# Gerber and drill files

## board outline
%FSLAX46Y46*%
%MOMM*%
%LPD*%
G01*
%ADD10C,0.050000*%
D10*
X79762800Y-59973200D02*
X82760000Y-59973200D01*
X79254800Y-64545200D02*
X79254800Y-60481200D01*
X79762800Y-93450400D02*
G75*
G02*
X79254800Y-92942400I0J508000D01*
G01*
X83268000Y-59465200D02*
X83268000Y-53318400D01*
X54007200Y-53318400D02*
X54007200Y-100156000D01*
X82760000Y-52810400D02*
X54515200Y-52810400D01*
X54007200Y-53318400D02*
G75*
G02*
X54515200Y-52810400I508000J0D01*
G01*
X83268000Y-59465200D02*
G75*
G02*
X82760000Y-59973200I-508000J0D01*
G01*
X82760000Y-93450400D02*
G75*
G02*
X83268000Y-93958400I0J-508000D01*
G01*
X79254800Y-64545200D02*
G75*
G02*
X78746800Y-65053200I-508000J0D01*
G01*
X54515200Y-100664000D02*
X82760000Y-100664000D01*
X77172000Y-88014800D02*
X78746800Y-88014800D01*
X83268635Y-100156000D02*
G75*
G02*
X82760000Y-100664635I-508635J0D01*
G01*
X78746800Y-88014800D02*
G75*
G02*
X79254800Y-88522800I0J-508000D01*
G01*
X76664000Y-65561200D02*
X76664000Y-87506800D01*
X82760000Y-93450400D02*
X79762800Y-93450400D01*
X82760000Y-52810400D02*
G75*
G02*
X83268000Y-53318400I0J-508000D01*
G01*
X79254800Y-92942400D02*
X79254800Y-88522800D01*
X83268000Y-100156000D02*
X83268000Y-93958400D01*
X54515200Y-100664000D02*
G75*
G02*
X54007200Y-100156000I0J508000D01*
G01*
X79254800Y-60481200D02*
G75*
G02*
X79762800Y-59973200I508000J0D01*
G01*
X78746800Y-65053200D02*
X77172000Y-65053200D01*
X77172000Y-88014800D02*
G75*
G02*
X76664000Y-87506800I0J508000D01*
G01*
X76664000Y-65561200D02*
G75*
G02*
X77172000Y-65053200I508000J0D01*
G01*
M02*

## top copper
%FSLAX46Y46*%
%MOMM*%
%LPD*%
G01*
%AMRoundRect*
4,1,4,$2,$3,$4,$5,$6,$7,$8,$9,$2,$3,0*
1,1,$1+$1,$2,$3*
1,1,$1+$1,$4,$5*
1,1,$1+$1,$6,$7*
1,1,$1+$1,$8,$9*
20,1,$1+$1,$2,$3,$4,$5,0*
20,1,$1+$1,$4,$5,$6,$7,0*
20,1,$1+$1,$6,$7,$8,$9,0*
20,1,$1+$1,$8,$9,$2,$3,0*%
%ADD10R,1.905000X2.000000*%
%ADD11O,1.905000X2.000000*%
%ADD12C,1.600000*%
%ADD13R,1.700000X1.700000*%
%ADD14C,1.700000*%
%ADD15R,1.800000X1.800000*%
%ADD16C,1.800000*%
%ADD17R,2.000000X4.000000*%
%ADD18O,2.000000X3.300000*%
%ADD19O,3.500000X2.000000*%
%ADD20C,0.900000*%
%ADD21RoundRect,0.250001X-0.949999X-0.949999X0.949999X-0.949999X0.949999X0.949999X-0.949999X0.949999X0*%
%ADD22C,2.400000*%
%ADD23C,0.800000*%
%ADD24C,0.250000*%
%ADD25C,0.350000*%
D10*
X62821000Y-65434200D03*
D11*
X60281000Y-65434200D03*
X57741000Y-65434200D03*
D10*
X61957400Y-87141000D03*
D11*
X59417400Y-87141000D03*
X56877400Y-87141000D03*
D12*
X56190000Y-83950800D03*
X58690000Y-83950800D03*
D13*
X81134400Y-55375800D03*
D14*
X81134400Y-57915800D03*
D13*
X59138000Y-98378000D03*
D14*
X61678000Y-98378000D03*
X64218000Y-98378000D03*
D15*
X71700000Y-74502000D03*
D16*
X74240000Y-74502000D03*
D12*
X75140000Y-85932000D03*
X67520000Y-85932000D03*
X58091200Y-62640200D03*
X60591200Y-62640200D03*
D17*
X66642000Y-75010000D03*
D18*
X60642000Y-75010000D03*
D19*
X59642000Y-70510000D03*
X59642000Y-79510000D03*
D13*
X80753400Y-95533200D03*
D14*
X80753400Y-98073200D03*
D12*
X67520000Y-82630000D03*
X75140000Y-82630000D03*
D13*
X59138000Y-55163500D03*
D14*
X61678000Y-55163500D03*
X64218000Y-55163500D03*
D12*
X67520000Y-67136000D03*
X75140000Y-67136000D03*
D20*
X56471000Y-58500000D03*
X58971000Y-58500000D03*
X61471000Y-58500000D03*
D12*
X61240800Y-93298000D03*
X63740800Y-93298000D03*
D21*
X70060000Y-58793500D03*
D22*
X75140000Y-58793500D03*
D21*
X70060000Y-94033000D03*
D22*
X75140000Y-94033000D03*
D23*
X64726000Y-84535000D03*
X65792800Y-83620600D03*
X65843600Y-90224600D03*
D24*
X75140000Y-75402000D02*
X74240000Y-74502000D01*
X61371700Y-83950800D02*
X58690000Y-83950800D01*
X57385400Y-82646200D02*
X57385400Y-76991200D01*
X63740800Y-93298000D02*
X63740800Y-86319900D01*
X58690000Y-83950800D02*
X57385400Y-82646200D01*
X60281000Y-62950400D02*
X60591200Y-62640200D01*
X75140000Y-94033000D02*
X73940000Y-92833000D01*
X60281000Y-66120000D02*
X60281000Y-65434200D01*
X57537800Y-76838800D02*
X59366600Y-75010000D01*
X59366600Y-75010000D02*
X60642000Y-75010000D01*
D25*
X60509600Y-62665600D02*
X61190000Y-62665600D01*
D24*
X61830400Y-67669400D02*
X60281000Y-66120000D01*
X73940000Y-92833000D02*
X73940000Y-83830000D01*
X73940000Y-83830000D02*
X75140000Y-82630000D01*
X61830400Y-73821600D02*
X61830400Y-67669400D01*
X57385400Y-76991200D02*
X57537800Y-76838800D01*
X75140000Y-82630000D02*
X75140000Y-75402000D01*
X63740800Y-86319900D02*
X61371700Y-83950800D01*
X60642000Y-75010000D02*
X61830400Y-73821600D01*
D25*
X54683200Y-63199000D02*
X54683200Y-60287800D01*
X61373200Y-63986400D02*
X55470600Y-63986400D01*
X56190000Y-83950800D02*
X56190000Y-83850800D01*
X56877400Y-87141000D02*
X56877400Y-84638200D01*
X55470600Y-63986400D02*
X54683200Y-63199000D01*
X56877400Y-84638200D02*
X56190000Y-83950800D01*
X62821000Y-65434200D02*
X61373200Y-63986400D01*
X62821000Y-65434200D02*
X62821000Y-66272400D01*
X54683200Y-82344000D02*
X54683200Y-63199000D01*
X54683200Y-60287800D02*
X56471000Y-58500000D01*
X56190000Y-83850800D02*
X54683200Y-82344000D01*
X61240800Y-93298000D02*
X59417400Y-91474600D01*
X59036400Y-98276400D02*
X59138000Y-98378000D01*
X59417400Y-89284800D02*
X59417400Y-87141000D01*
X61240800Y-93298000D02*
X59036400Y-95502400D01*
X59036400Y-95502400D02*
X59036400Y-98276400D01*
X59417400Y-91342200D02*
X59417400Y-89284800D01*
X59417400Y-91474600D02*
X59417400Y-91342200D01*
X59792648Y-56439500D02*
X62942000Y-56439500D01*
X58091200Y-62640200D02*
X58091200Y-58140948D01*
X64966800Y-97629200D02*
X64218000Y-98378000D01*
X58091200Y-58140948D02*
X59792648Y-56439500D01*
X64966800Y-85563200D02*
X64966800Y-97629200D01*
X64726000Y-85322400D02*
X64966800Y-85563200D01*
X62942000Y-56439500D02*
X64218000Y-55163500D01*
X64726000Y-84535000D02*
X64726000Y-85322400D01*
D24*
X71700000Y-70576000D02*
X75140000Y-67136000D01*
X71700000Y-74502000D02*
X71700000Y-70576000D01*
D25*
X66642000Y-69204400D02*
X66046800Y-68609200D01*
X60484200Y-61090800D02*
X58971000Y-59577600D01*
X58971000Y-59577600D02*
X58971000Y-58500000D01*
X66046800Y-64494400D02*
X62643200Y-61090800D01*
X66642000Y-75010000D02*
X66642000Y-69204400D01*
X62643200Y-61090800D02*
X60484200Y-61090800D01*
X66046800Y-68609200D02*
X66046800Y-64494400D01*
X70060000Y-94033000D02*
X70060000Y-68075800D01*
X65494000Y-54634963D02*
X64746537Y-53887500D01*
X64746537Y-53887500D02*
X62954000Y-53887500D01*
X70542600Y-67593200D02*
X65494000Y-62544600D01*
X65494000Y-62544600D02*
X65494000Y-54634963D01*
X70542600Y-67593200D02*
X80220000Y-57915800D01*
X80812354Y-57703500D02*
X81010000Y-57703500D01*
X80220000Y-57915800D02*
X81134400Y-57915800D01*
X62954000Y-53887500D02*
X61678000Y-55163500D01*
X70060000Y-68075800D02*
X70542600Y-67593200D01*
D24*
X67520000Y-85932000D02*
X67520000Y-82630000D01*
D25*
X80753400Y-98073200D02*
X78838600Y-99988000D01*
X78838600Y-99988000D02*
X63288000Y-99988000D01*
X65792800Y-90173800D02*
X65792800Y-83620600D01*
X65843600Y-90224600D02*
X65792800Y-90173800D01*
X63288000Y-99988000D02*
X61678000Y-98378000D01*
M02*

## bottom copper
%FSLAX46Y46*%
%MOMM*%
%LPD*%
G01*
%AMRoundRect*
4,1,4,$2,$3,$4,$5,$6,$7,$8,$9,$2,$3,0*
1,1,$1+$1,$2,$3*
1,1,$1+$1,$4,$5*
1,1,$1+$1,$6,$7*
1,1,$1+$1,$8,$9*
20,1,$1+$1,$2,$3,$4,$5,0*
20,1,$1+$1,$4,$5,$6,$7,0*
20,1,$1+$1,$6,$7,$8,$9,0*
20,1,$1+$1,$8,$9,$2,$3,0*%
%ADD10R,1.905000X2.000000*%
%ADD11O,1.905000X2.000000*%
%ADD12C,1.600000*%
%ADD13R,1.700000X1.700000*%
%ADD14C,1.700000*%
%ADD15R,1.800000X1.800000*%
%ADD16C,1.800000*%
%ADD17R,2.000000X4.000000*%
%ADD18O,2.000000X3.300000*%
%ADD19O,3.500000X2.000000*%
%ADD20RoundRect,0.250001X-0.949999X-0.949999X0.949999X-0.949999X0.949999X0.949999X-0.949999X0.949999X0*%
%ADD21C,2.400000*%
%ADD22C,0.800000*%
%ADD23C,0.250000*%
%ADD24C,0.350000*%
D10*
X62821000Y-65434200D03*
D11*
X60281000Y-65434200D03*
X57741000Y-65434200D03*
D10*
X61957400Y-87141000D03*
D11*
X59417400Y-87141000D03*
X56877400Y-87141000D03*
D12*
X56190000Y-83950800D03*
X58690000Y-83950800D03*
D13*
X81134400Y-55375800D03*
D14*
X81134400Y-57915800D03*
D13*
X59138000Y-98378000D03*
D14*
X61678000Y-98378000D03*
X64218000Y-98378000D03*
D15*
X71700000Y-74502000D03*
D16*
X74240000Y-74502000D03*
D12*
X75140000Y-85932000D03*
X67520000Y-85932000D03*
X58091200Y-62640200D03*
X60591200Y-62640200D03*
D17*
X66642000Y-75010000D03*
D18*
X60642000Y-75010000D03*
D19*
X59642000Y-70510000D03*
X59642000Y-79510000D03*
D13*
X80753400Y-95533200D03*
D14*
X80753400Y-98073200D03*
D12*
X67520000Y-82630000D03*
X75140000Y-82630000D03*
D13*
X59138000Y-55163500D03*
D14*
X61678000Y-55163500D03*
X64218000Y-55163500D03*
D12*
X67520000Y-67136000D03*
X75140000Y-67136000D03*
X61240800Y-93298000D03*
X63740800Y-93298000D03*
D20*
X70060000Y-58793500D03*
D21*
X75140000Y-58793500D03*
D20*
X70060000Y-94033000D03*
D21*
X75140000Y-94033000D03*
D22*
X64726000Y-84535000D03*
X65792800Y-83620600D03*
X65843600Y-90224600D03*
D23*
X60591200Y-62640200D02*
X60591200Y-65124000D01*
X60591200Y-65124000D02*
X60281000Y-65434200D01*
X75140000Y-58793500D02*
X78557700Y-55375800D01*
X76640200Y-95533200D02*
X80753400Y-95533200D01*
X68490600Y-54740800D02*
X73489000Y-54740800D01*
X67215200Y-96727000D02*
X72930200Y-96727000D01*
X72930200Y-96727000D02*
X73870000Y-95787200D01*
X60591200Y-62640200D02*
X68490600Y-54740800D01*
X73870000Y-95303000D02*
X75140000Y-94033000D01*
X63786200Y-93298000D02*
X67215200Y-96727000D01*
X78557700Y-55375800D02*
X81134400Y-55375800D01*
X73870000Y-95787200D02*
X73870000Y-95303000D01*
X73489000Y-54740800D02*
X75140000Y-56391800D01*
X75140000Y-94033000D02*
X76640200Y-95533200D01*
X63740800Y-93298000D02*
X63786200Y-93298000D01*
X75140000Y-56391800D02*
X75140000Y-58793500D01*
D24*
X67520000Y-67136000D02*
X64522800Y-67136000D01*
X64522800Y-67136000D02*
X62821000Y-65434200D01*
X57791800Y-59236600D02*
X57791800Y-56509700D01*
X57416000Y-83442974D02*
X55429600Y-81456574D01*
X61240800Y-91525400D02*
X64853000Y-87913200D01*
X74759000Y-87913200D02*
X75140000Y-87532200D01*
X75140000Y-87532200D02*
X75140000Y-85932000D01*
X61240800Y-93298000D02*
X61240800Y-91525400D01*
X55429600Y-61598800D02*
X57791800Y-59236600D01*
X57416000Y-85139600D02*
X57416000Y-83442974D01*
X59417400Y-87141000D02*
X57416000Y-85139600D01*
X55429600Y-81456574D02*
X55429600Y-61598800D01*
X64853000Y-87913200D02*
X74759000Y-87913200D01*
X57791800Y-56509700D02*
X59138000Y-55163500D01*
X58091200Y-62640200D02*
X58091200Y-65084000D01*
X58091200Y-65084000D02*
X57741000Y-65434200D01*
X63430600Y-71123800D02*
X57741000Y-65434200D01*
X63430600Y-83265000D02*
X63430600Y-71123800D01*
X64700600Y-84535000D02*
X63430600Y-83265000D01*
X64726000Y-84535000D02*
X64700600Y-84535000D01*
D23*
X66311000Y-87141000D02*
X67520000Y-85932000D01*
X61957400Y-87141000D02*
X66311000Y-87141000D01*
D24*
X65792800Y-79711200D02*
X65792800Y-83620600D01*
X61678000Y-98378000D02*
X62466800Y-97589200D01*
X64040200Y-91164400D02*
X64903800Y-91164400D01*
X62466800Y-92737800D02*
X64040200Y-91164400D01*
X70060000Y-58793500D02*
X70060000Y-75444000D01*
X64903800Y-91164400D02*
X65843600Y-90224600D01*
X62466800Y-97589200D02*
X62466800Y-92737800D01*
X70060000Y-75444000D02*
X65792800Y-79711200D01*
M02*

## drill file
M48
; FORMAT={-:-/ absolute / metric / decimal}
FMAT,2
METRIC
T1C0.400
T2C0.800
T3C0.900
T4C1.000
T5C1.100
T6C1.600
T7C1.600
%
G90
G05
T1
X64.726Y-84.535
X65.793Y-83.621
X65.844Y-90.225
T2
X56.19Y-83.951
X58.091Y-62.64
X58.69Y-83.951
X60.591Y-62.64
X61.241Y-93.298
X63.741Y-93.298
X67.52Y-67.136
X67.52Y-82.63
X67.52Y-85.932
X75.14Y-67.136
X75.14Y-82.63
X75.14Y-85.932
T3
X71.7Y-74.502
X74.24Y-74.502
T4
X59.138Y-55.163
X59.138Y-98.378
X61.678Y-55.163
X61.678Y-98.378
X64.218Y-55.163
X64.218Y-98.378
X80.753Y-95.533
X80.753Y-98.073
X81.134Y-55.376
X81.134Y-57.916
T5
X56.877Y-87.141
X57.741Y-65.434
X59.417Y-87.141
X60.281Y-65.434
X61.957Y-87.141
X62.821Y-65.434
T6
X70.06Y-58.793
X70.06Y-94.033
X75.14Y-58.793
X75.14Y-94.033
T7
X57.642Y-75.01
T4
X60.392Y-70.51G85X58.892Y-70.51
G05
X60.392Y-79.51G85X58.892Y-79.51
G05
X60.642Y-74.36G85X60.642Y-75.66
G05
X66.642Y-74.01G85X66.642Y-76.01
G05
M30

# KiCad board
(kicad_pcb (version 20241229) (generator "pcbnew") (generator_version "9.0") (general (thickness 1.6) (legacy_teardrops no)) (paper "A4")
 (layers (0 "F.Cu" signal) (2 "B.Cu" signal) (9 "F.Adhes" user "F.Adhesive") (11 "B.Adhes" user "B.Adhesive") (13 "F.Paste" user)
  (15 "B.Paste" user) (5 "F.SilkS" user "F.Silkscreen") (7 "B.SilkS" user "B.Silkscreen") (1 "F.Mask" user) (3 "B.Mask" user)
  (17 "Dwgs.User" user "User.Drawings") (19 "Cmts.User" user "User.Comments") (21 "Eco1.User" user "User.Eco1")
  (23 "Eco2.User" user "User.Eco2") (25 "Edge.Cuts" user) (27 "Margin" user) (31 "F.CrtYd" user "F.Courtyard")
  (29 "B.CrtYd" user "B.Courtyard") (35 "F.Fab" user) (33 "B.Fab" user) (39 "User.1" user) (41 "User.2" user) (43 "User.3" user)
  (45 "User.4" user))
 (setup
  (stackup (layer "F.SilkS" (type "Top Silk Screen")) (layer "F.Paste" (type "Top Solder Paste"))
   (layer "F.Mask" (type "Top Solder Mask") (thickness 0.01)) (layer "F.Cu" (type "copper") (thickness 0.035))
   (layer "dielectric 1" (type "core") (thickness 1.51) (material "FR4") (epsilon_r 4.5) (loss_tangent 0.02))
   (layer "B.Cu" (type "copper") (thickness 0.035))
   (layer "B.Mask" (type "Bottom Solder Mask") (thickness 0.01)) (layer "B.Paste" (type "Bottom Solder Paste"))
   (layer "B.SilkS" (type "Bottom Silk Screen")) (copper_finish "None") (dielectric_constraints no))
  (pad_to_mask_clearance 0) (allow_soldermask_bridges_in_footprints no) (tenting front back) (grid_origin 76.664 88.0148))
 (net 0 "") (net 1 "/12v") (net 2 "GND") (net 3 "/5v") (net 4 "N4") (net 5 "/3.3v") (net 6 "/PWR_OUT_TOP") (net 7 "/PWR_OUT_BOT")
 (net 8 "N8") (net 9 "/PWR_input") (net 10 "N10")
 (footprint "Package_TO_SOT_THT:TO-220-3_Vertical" (layer "F.Cu") (at 62.821 65.4342 180)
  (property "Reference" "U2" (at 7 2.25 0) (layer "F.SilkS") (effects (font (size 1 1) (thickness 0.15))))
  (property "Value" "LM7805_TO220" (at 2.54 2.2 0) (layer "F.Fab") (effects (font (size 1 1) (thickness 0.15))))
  (pad "1" thru_hole rect (at 0 0 180) (size 1.905 2) (drill 1.1) (layers "*.Cu" "*.Mask") (remove_unused_layers no) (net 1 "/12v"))
  (pad "2" thru_hole oval (at 2.54 0 180) (size 1.905 2) (drill 1.1) (layers "*.Cu" "*.Mask") (remove_unused_layers no) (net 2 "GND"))
  (pad "3" thru_hole oval (at 5.08 0 180) (size 1.905 2) (drill 1.1) (layers "*.Cu" "*.Mask") (remove_unused_layers no) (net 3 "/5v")))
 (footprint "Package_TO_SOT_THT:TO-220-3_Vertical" (layer "F.Cu") (at 61.9574 87.141 180)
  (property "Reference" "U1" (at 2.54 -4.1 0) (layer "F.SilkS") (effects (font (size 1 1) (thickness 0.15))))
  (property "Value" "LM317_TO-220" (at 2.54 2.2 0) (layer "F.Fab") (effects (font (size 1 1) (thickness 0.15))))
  (pad "1" thru_hole rect (at 0 0 180) (size 1.905 2) (drill 1.1) (layers "*.Cu" "*.Mask") (remove_unused_layers no) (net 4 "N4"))
  (pad "2" thru_hole oval (at 2.54 0 180) (size 1.905 2) (drill 1.1) (layers "*.Cu" "*.Mask") (remove_unused_layers no) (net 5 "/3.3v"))
  (pad "3" thru_hole oval (at 5.08 0 180) (size 1.905 2) (drill 1.1) (layers "*.Cu" "*.Mask") (remove_unused_layers no) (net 1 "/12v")))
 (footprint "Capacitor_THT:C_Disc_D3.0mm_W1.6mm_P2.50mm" (layer "F.Cu") (at 56.19 83.9508)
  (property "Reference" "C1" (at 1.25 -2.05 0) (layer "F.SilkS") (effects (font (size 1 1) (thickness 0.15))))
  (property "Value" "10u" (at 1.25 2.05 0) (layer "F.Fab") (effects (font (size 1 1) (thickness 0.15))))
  (pad "1" thru_hole circle (at 0 0) (size 1.6 1.6) (drill 0.8) (layers "*.Cu" "*.Mask") (remove_unused_layers no) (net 1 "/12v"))
  (pad "2" thru_hole circle (at 2.5 0) (size 1.6 1.6) (drill 0.8) (layers "*.Cu" "*.Mask") (remove_unused_layers no) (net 2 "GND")))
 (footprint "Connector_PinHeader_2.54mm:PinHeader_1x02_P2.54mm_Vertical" (layer "F.Cu") (at 81.1344 55.3758)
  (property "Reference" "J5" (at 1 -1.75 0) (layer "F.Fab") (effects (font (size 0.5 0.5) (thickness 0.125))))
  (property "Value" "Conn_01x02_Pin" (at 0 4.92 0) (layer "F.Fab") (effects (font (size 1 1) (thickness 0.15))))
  (pad "1" thru_hole rect (at 0 0) (size 1.7 1.7) (drill 1) (layers "*.Cu" "*.Mask") (remove_unused_layers no) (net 2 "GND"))
  (pad "2" thru_hole circle (at 0 2.54) (size 1.7 1.7) (drill 1) (layers "*.Cu" "*.Mask") (remove_unused_layers no) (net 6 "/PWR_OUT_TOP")))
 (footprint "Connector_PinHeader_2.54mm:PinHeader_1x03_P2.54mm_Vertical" (layer "F.Cu") (at 59.138 98.378 90)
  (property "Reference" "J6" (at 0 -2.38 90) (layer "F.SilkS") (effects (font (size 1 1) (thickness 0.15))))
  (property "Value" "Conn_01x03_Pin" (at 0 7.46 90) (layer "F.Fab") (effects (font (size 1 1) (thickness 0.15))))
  (pad "1" thru_hole rect (at 0 0 90) (size 1.7 1.7) (drill 1) (layers "*.Cu" "*.Mask") (remove_unused_layers no) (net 5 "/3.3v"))
  (pad "2" thru_hole circle (at 0 2.54 90) (size 1.7 1.7) (drill 1) (layers "*.Cu" "*.Mask") (remove_unused_layers no)
   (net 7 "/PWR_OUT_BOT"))
  (pad "3" thru_hole circle (at 0 5.08 90) (size 1.7 1.7) (drill 1) (layers "*.Cu" "*.Mask") (remove_unused_layers no) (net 3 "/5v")))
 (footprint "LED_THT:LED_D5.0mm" (layer "F.Cu") (at 71.7 74.502)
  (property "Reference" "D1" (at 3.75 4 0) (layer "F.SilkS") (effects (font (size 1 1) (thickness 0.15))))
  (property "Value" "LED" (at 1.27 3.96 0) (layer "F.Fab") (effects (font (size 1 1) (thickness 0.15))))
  (pad "1" thru_hole rect (at 0 0) (size 1.8 1.8) (drill 0.9) (layers "*.Cu" "*.Mask") (remove_unused_layers no) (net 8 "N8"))
  (pad "2" thru_hole circle (at 2.54 0) (size 1.8 1.8) (drill 0.9) (layers "*.Cu" "*.Mask") (remove_unused_layers no) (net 2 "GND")))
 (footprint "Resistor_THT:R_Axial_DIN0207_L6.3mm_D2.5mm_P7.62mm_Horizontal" (layer "F.Cu") (at 75.14 85.932 180)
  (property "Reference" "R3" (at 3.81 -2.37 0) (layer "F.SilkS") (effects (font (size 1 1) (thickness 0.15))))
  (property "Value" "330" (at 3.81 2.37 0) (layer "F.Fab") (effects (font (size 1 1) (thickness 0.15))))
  (pad "1" thru_hole circle (at 0 0 180) (size 1.6 1.6) (drill 0.8) (layers "*.Cu" "*.Mask") (remove_unused_layers no) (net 5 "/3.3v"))
  (pad "2" thru_hole circle (at 7.62 0 180) (size 1.6 1.6) (drill 0.8) (layers "*.Cu" "*.Mask") (remove_unused_layers no) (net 4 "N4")))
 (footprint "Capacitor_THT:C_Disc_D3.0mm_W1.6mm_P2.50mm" (layer "F.Cu") (at 58.0912 62.6402)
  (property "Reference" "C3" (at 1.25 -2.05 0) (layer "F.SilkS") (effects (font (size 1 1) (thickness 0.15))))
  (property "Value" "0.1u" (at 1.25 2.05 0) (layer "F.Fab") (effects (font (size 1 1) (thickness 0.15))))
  (pad "1" thru_hole circle (at 0 0) (size 1.6 1.6) (drill 0.8) (layers "*.Cu" "*.Mask") (remove_unused_layers no) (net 3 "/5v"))
  (pad "2" thru_hole circle (at 2.5 0) (size 1.6 1.6) (drill 0.8) (layers "*.Cu" "*.Mask") (remove_unused_layers no) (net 2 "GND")))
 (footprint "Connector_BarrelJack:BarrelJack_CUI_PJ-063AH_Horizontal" (layer "F.Cu") (at 66.642 75.01 -90)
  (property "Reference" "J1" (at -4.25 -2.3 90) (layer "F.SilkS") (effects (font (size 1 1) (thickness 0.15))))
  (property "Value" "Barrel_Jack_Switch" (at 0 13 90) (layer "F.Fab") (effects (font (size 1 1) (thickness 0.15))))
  (pad "" np_thru_hole circle (at 0 9 270) (size 1.6 1.6) (drill 1.6) (layers "*.Cu" "*.Mask"))
  (pad "1" thru_hole rect (at 0 0 270) (size 4 2) (drill oval 3 1) (layers "*.Cu" "*.Mask") (remove_unused_layers no) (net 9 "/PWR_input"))
  (pad "2" thru_hole oval (at 0 6 270) (size 3.3 2) (drill oval 2.3 1) (layers "*.Cu" "*.Mask") (remove_unused_layers no) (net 2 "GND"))
  (pad "MP" thru_hole oval (at -4.5 7 270) (size 2 3.5) (drill oval 1 2.5) (layers "*.Cu" "*.Mask") (remove_unused_layers no))
  (pad "MP" thru_hole oval (at 4.5 7 270) (size 2 3.5) (drill oval 1 2.5) (layers "*.Cu" "*.Mask") (remove_unused_layers no)))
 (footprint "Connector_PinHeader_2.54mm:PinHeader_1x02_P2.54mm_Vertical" (layer "F.Cu") (at 80.7534 95.5332)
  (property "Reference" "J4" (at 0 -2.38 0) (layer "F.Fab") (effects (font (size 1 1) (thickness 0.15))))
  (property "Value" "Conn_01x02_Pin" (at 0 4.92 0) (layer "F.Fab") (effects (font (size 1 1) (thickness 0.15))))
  (pad "1" thru_hole rect (at 0 0) (size 1.7 1.7) (drill 1) (layers "*.Cu" "*.Mask") (remove_unused_layers no) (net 2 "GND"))
  (pad "2" thru_hole circle (at 0 2.54) (size 1.7 1.7) (drill 1) (layers "*.Cu" "*.Mask") (remove_unused_layers no) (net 7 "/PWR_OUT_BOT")))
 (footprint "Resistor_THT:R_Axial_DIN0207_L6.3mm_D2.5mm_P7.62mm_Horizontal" (layer "F.Cu") (at 67.52 82.63)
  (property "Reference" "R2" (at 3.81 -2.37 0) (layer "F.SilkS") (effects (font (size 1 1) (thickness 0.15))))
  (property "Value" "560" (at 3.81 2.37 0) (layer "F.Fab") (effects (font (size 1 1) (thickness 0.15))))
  (pad "1" thru_hole circle (at 0 0) (size 1.6 1.6) (drill 0.8) (layers "*.Cu" "*.Mask") (remove_unused_layers no) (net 4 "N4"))
  (pad "2" thru_hole circle (at 7.62 0) (size 1.6 1.6) (drill 0.8) (layers "*.Cu" "*.Mask") (remove_unused_layers no) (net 2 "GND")))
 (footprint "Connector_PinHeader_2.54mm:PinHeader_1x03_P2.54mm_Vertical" (layer "F.Cu") (at 59.138 55.1635 90)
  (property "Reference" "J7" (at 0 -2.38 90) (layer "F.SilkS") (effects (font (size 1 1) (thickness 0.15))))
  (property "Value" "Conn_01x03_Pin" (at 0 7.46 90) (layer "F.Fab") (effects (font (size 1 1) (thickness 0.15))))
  (pad "1" thru_hole rect (at 0 0 90) (size 1.7 1.7) (drill 1) (layers "*.Cu" "*.Mask") (remove_unused_layers no) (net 5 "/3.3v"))
  (pad "2" thru_hole circle (at 0 2.54 90) (size 1.7 1.7) (drill 1) (layers "*.Cu" "*.Mask") (remove_unused_layers no)
   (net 6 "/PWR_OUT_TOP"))
  (pad "3" thru_hole circle (at 0 5.08 90) (size 1.7 1.7) (drill 1) (layers "*.Cu" "*.Mask") (remove_unused_layers no) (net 3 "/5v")))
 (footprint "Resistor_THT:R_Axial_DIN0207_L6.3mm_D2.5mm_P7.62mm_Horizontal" (layer "F.Cu") (at 67.52 67.136)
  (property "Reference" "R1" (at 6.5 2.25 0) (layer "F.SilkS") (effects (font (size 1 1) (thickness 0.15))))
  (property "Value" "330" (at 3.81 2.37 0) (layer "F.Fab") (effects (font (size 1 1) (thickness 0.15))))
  (pad "1" thru_hole circle (at 0 0) (size 1.6 1.6) (drill 0.8) (layers "*.Cu" "*.Mask") (remove_unused_layers no) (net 1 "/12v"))
  (pad "2" thru_hole circle (at 7.62 0) (size 1.6 1.6) (drill 0.8) (layers "*.Cu" "*.Mask") (remove_unused_layers no) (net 8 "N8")))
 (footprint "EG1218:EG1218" (layer "F.Cu") (at 50.471 58.5 90)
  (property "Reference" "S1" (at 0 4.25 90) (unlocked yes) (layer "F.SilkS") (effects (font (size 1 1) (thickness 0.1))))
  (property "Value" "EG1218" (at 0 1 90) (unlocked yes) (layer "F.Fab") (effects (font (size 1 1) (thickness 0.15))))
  (pad "1" connect circle (at 0 6 90) (size 0.9 0.9) (layers "F.Cu" "F.Mask") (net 1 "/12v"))
  (pad "2" connect circle (at 0 8.5 90) (size 0.9 0.9) (layers "F.Cu" "F.Mask") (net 9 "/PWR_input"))
  (pad "3" connect circle (at 0 11 90) (size 0.9 0.9) (layers "F.Cu" "F.Mask") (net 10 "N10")))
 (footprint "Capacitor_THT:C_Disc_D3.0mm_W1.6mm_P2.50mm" (layer "F.Cu") (at 61.2408 93.298)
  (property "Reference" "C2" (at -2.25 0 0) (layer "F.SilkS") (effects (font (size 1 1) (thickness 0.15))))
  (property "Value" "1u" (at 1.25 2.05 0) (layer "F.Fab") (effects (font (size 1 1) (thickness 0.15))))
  (pad "1" thru_hole circle (at 0 0) (size 1.6 1.6) (drill 0.8) (layers "*.Cu" "*.Mask") (remove_unused_layers no) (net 5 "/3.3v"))
  (pad "2" thru_hole circle (at 2.5 0) (size 1.6 1.6) (drill 0.8) (layers "*.Cu" "*.Mask") (remove_unused_layers no) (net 2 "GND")))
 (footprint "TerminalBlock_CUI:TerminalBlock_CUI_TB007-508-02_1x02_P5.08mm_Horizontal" (layer "F.Cu") (at 70.06 58.7935)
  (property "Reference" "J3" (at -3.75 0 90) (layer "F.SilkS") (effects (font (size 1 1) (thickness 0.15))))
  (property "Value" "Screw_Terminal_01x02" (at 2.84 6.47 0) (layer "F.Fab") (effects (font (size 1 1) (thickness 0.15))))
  (pad "1" thru_hole roundrect (at 0 0) (size 2.4 2.4) (drill 1.6) (layers "*.Cu" "*.Mask") (remove_unused_layers no)
   (roundrect_rratio 0.104167) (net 7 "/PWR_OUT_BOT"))
  (pad "2" thru_hole circle (at 5.08 0) (size 2.4 2.4) (drill 1.6) (layers "*.Cu" "*.Mask") (remove_unused_layers no) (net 2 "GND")))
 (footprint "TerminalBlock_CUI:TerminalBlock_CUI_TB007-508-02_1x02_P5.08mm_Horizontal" (layer "F.Cu") (at 70.06 94.033)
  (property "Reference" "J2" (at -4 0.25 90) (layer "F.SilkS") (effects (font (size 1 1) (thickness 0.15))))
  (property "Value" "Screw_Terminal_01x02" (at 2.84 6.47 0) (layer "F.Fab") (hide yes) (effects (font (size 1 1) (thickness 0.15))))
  (pad "1" thru_hole roundrect (at 0 0) (size 2.4 2.4) (drill 1.6) (layers "*.Cu" "*.Mask") (remove_unused_layers no)
   (roundrect_rratio 0.104167) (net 6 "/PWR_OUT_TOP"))
  (pad "2" thru_hole circle (at 5.08 0) (size 2.4 2.4) (drill 1.6) (layers "*.Cu" "*.Mask") (remove_unused_layers no) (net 2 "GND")))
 (gr_line (start 79.7628 59.9732) (end 82.76 59.9732) (stroke (width 0.05) (type default)) (layer "Edge.Cuts"))
 (gr_line (start 79.2548 64.5452) (end 79.2548 60.4812) (stroke (width 0.05) (type default)) (layer "Edge.Cuts"))
 (gr_arc (start 79.7628 93.4504) (mid 79.40359 93.30161) (end 79.2548 92.9424) (stroke (width 0.05) (type default)) (layer "Edge.Cuts"))
 (gr_line (start 83.268 59.4652) (end 83.268 53.3184) (stroke (width 0.05) (type default)) (layer "Edge.Cuts"))
 (gr_line (start 54.0072 53.3184) (end 54.0072 100.156) (stroke (width 0.05) (type default)) (layer "Edge.Cuts"))
 (gr_line (start 82.76 52.8104) (end 54.5152 52.8104) (stroke (width 0.05) (type default)) (layer "Edge.Cuts"))
 (gr_arc (start 54.0072 53.3184) (mid 54.15599 52.95919) (end 54.5152 52.8104) (stroke (width 0.05) (type default)) (layer "Edge.Cuts"))
 (gr_arc (start 83.268 59.4652) (mid 83.11921 59.82441) (end 82.76 59.9732) (stroke (width 0.05) (type default)) (layer "Edge.Cuts"))
 (gr_arc (start 82.76 93.4504) (mid 83.11921 93.59919) (end 83.268 93.9584) (stroke (width 0.05) (type default)) (layer "Edge.Cuts"))
 (gr_arc (start 79.2548 64.5452) (mid 79.10601 64.90441) (end 78.7468 65.0532) (stroke (width 0.05) (type default)) (layer "Edge.Cuts"))
 (gr_line (start 54.5152 100.664) (end 82.76 100.664) (stroke (width 0.05) (type default)) (layer "Edge.Cuts"))
 (gr_line (start 77.172 88.0148) (end 78.7468 88.0148) (stroke (width 0.05) (type default)) (layer "Edge.Cuts"))
 (gr_arc (start 83.268635 100.156) (mid 83.119659 100.515659) (end 82.76 100.664635) (stroke (width 0.05) (type default))
  (layer "Edge.Cuts"))
 (gr_arc (start 78.7468 88.0148) (mid 79.10601 88.16359) (end 79.2548 88.5228) (stroke (width 0.05) (type default)) (layer "Edge.Cuts"))
 (gr_line (start 76.664 65.5612) (end 76.664 87.5068) (stroke (width 0.05) (type default)) (layer "Edge.Cuts"))
 (gr_line (start 82.76 93.4504) (end 79.7628 93.4504) (stroke (width 0.05) (type default)) (layer "Edge.Cuts"))
 (gr_arc (start 82.76 52.8104) (mid 83.11921 52.95919) (end 83.268 53.3184) (stroke (width 0.05) (type default)) (layer "Edge.Cuts"))
 (gr_line (start 79.2548 92.9424) (end 79.2548 88.5228) (stroke (width 0.05) (type default)) (layer "Edge.Cuts"))
 (gr_line (start 83.268 100.156) (end 83.268 93.9584) (stroke (width 0.05) (type default)) (layer "Edge.Cuts"))
 (gr_arc (start 54.5152 100.664) (mid 54.15599 100.51521) (end 54.0072 100.156) (stroke (width 0.05) (type default)) (layer "Edge.Cuts"))
 (gr_arc (start 79.2548 60.4812) (mid 79.40359 60.12199) (end 79.7628 59.9732) (stroke (width 0.05) (type default)) (layer "Edge.Cuts"))
 (gr_line (start 78.7468 65.0532) (end 77.172 65.0532) (stroke (width 0.05) (type default)) (layer "Edge.Cuts"))
 (gr_arc (start 77.172 88.0148) (mid 76.81279 87.86601) (end 76.664 87.5068) (stroke (width 0.05) (type default)) (layer "Edge.Cuts"))
 (gr_arc (start 76.664 65.5612) (mid 76.81279 65.20199) (end 77.172 65.0532) (stroke (width 0.05) (type default)) (layer "Edge.Cuts"))
 (segment (start 75.14 75.402) (end 74.24 74.502) (width 0.25) (layer "F.Cu") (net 2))
 (segment (start 61.3717 83.9508) (end 58.69 83.9508) (width 0.25) (layer "F.Cu") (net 2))
 (segment (start 57.3854 82.6462) (end 57.3854 76.9912) (width 0.25) (layer "F.Cu") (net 2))
 (segment (start 63.7408 93.298) (end 63.7408 86.3199) (width 0.25) (layer "F.Cu") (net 2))
 (segment (start 58.69 83.9508) (end 57.3854 82.6462) (width 0.25) (layer "F.Cu") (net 2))
 (segment (start 60.281 62.9504) (end 60.5912 62.6402) (width 0.25) (layer "F.Cu") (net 2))
 (segment (start 75.14 94.033) (end 73.94 92.833) (width 0.25) (layer "F.Cu") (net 2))
 (segment (start 60.281 66.12) (end 60.281 65.4342) (width 0.25) (layer "F.Cu") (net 2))
 (segment (start 57.5378 76.8388) (end 59.3666 75.01) (width 0.25) (layer "F.Cu") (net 2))
 (segment (start 59.3666 75.01) (end 60.642 75.01) (width 0.25) (layer "F.Cu") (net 2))
 (segment (start 60.5096 62.6656) (end 61.19 62.6656) (width 0.35) (layer "F.Cu") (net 2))
 (segment (start 61.8304 67.6694) (end 60.281 66.12) (width 0.25) (layer "F.Cu") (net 2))
 (segment (start 73.94 92.833) (end 73.94 83.83) (width 0.25) (layer "F.Cu") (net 2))
 (segment (start 73.94 83.83) (end 75.14 82.63) (width 0.25) (layer "F.Cu") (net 2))
 (segment (start 61.8304 73.8216) (end 61.8304 67.6694) (width 0.25) (layer "F.Cu") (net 2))
 (segment (start 57.3854 76.9912) (end 57.5378 76.8388) (width 0.25) (layer "F.Cu") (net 2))
 (segment (start 75.14 82.63) (end 75.14 75.402) (width 0.25) (layer "F.Cu") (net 2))
 (segment (start 63.7408 86.3199) (end 61.3717 83.9508) (width 0.25) (layer "F.Cu") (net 2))
 (segment (start 60.642 75.01) (end 61.8304 73.8216) (width 0.25) (layer "F.Cu") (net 2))
 (segment (start 60.5912 62.6402) (end 60.5912 65.124) (width 0.25) (layer "B.Cu") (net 2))
 (segment (start 60.5912 65.124) (end 60.281 65.4342) (width 0.25) (layer "B.Cu") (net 2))
 (segment (start 75.14 58.7935) (end 78.5577 55.3758) (width 0.25) (layer "B.Cu") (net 2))
 (segment (start 76.6402 95.5332) (end 80.7534 95.5332) (width 0.25) (layer "B.Cu") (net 2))
 (segment (start 68.4906 54.7408) (end 73.489 54.7408) (width 0.25) (layer "B.Cu") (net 2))
 (segment (start 67.2152 96.727) (end 72.9302 96.727) (width 0.25) (layer "B.Cu") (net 2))
 (segment (start 72.9302 96.727) (end 73.87 95.7872) (width 0.25) (layer "B.Cu") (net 2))
 (segment (start 60.5912 62.6402) (end 68.4906 54.7408) (width 0.25) (layer "B.Cu") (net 2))
 (segment (start 73.87 95.303) (end 75.14 94.033) (width 0.25) (layer "B.Cu") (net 2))
 (segment (start 63.7862 93.298) (end 67.2152 96.727) (width 0.25) (layer "B.Cu") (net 2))
 (segment (start 78.5577 55.3758) (end 81.1344 55.3758) (width 0.25) (layer "B.Cu") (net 2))
 (segment (start 73.87 95.7872) (end 73.87 95.303) (width 0.25) (layer "B.Cu") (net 2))
 (segment (start 73.489 54.7408) (end 75.14 56.3918) (width 0.25) (layer "B.Cu") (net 2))
 (segment (start 75.14 94.033) (end 76.6402 95.5332) (width 0.25) (layer "B.Cu") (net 2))
 (segment (start 63.7408 93.298) (end 63.7862 93.298) (width 0.25) (layer "B.Cu") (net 2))
 (segment (start 75.14 56.3918) (end 75.14 58.7935) (width 0.25) (layer "B.Cu") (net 2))
 (segment (start 54.6832 63.199) (end 54.6832 60.2878) (width 0.35) (layer "F.Cu") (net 1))
 (segment (start 61.3732 63.9864) (end 55.4706 63.9864) (width 0.35) (layer "F.Cu") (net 1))
 (segment (start 56.19 83.9508) (end 56.19 83.8508) (width 0.35) (layer "F.Cu") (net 1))
 (segment (start 56.8774 87.141) (end 56.8774 84.6382) (width 0.35) (layer "F.Cu") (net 1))
 (segment (start 55.4706 63.9864) (end 54.6832 63.199) (width 0.35) (layer "F.Cu") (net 1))
 (segment (start 56.8774 84.6382) (end 56.19 83.9508) (width 0.35) (layer "F.Cu") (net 1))
 (segment (start 62.821 65.4342) (end 61.3732 63.9864) (width 0.35) (layer "F.Cu") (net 1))
 (segment (start 62.821 65.4342) (end 62.821 66.2724) (width 0.35) (layer "F.Cu") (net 1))
 (segment (start 54.6832 82.344) (end 54.6832 63.199) (width 0.35) (layer "F.Cu") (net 1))
 (segment (start 54.6832 60.2878) (end 56.471 58.5) (width 0.35) (layer "F.Cu") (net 1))
 (segment (start 56.19 83.8508) (end 54.6832 82.344) (width 0.35) (layer "F.Cu") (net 1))
 (segment (start 67.52 67.136) (end 64.5228 67.136) (width 0.35) (layer "B.Cu") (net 1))
 (segment (start 64.5228 67.136) (end 62.821 65.4342) (width 0.35) (layer "B.Cu") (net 1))
 (segment (start 61.2408 93.298) (end 59.4174 91.4746) (width 0.35) (layer "F.Cu") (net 5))
 (segment (start 59.0364 98.2764) (end 59.138 98.378) (width 0.35) (layer "F.Cu") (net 5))
 (segment (start 59.4174 89.2848) (end 59.4174 87.141) (width 0.35) (layer "F.Cu") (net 5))
 (segment (start 61.2408 93.298) (end 59.0364 95.5024) (width 0.35) (layer "F.Cu") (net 5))
 (segment (start 59.0364 95.5024) (end 59.0364 98.2764) (width 0.35) (layer "F.Cu") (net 5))
 (segment (start 59.4174 91.3422) (end 59.4174 89.2848) (width 0.35) (layer "F.Cu") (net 5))
 (segment (start 59.4174 91.4746) (end 59.4174 91.3422) (width 0.35) (layer "F.Cu") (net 5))
 (segment (start 57.7918 59.2366) (end 57.7918 56.5097) (width 0.35) (layer "B.Cu") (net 5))
 (segment (start 57.416 83.442974) (end 55.4296 81.456574) (width 0.35) (layer "B.Cu") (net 5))
 (segment (start 61.2408 91.5254) (end 64.853 87.9132) (width 0.35) (layer "B.Cu") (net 5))
 (segment (start 74.759 87.9132) (end 75.14 87.5322) (width 0.35) (layer "B.Cu") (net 5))
 (segment (start 75.14 87.5322) (end 75.14 85.932) (width 0.35) (layer "B.Cu") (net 5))
 (segment (start 61.2408 93.298) (end 61.2408 91.5254) (width 0.35) (layer "B.Cu") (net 5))
 (segment (start 55.4296 61.5988) (end 57.7918 59.2366) (width 0.35) (layer "B.Cu") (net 5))
 (segment (start 57.416 85.1396) (end 57.416 83.442974) (width 0.35) (layer "B.Cu") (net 5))
 (segment (start 59.4174 87.141) (end 57.416 85.1396) (width 0.35) (layer "B.Cu") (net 5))
 (segment (start 55.4296 81.456574) (end 55.4296 61.5988) (width 0.35) (layer "B.Cu") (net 5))
 (segment (start 64.853 87.9132) (end 74.759 87.9132) (width 0.35) (layer "B.Cu") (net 5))
 (segment (start 57.7918 56.5097) (end 59.138 55.1635) (width 0.35) (layer "B.Cu") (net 5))
 (segment (start 59.792648 56.4395) (end 62.942 56.4395) (width 0.35) (layer "F.Cu") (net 3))
 (segment (start 58.0912 62.6402) (end 58.0912 58.140948) (width 0.35) (layer "F.Cu") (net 3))
 (segment (start 64.9668 97.6292) (end 64.218 98.378) (width 0.35) (layer "F.Cu") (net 3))
 (segment (start 58.0912 58.140948) (end 59.792648 56.4395) (width 0.35) (layer "F.Cu") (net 3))
 (segment (start 64.9668 85.5632) (end 64.9668 97.6292) (width 0.35) (layer "F.Cu") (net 3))
 (segment (start 64.726 85.3224) (end 64.9668 85.5632) (width 0.35) (layer "F.Cu") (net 3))
 (segment (start 62.942 56.4395) (end 64.218 55.1635) (width 0.35) (layer "F.Cu") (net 3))
 (segment (start 64.726 84.535) (end 64.726 85.3224) (width 0.35) (layer "F.Cu") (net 3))
 (via (at 64.726 84.535) (size 0.8) (drill 0.4) (layers "F.Cu" "B.Cu") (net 3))
 (segment (start 58.0912 62.6402) (end 58.0912 65.084) (width 0.35) (layer "B.Cu") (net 3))
 (segment (start 58.0912 65.084) (end 57.741 65.4342) (width 0.35) (layer "B.Cu") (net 3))
 (segment (start 63.4306 71.1238) (end 57.741 65.4342) (width 0.35) (layer "B.Cu") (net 3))
 (segment (start 63.4306 83.265) (end 63.4306 71.1238) (width 0.35) (layer "B.Cu") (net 3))
 (segment (start 64.7006 84.535) (end 63.4306 83.265) (width 0.35) (layer "B.Cu") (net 3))
 (segment (start 64.726 84.535) (end 64.7006 84.535) (width 0.35) (layer "B.Cu") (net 3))
 (segment (start 71.7 70.576) (end 75.14 67.136) (width 0.25) (layer "F.Cu") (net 8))
 (segment (start 71.7 74.502) (end 71.7 70.576) (width 0.25) (layer "F.Cu") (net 8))
 (segment (start 66.642 69.2044) (end 66.0468 68.6092) (width 0.35) (layer "F.Cu") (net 9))
 (segment (start 60.4842 61.0908) (end 58.971 59.5776) (width 0.35) (layer "F.Cu") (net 9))
 (segment (start 58.971 59.5776) (end 58.971 58.5) (width 0.35) (layer "F.Cu") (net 9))
 (segment (start 66.0468 64.4944) (end 62.6432 61.0908) (width 0.35) (layer "F.Cu") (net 9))
 (segment (start 66.642 75.01) (end 66.642 69.2044) (width 0.35) (layer "F.Cu") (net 9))
 (segment (start 62.6432 61.0908) (end 60.4842 61.0908) (width 0.35) (layer "F.Cu") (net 9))
 (segment (start 66.0468 68.6092) (end 66.0468 64.4944) (width 0.35) (layer "F.Cu") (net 9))
 (segment (start 70.06 94.033) (end 70.06 68.0758) (width 0.35) (layer "F.Cu") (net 6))
 (segment (start 65.494 54.634963) (end 64.746537 53.8875) (width 0.35) (layer "F.Cu") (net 6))
 (segment (start 64.746537 53.8875) (end 62.954 53.8875) (width 0.35) (layer "F.Cu") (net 6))
 (segment (start 70.5426 67.5932) (end 65.494 62.5446) (width 0.35) (layer "F.Cu") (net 6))
 (segment (start 65.494 62.5446) (end 65.494 54.634963) (width 0.35) (layer "F.Cu") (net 6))
 (segment (start 70.5426 67.5932) (end 80.22 57.9158) (width 0.35) (layer "F.Cu") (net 6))
 (segment (start 80.812354 57.7035) (end 81.01 57.7035) (width 0.35) (layer "F.Cu") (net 6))
 (segment (start 80.22 57.9158) (end 81.1344 57.9158) (width 0.35) (layer "F.Cu") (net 6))
 (segment (start 62.954 53.8875) (end 61.678 55.1635) (width 0.35) (layer "F.Cu") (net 6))
 (segment (start 70.06 68.0758) (end 70.5426 67.5932) (width 0.35) (layer "F.Cu") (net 6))
 (segment (start 67.52 85.932) (end 67.52 82.63) (width 0.25) (layer "F.Cu") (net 4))
 (segment (start 66.311 87.141) (end 67.52 85.932) (width 0.25) (layer "B.Cu") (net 4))
 (segment (start 61.9574 87.141) (end 66.311 87.141) (width 0.25) (layer "B.Cu") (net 4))
 (segment (start 80.7534 98.0732) (end 78.8386 99.988) (width 0.35) (layer "F.Cu") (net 7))
 (segment (start 78.8386 99.988) (end 63.288 99.988) (width 0.35) (layer "F.Cu") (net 7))
 (segment (start 65.7928 90.1738) (end 65.7928 83.6206) (width 0.35) (layer "F.Cu") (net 7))
 (segment (start 65.8436 90.2246) (end 65.7928 90.1738) (width 0.35) (layer "F.Cu") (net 7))
 (segment (start 63.288 99.988) (end 61.678 98.378) (width 0.35) (layer "F.Cu") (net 7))
 (via (at 65.7928 83.6206) (size 0.8) (drill 0.4) (layers "F.Cu" "B.Cu") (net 7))
 (via (at 65.8436 90.2246) (size 0.8) (drill 0.4) (layers "F.Cu" "B.Cu") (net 7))
 (segment (start 65.7928 79.7112) (end 65.7928 83.6206) (width 0.35) (layer "B.Cu") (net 7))
 (segment (start 61.678 98.378) (end 62.4668 97.5892) (width 0.35) (layer "B.Cu") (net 7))
 (segment (start 64.0402 91.1644) (end 64.9038 91.1644) (width 0.35) (layer "B.Cu") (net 7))
 (segment (start 62.4668 92.7378) (end 64.0402 91.1644) (width 0.35) (layer "B.Cu") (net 7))
 (segment (start 70.06 58.7935) (end 70.06 75.444) (width 0.35) (layer "B.Cu") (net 7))
 (segment (start 64.9038 91.1644) (end 65.8436 90.2246) (width 0.35) (layer "B.Cu") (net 7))
 (segment (start 62.4668 97.5892) (end 62.4668 92.7378) (width 0.35) (layer "B.Cu") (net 7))
 (segment (start 70.06 75.444) (end 65.7928 79.7112) (width 0.35) (layer "B.Cu") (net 7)))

